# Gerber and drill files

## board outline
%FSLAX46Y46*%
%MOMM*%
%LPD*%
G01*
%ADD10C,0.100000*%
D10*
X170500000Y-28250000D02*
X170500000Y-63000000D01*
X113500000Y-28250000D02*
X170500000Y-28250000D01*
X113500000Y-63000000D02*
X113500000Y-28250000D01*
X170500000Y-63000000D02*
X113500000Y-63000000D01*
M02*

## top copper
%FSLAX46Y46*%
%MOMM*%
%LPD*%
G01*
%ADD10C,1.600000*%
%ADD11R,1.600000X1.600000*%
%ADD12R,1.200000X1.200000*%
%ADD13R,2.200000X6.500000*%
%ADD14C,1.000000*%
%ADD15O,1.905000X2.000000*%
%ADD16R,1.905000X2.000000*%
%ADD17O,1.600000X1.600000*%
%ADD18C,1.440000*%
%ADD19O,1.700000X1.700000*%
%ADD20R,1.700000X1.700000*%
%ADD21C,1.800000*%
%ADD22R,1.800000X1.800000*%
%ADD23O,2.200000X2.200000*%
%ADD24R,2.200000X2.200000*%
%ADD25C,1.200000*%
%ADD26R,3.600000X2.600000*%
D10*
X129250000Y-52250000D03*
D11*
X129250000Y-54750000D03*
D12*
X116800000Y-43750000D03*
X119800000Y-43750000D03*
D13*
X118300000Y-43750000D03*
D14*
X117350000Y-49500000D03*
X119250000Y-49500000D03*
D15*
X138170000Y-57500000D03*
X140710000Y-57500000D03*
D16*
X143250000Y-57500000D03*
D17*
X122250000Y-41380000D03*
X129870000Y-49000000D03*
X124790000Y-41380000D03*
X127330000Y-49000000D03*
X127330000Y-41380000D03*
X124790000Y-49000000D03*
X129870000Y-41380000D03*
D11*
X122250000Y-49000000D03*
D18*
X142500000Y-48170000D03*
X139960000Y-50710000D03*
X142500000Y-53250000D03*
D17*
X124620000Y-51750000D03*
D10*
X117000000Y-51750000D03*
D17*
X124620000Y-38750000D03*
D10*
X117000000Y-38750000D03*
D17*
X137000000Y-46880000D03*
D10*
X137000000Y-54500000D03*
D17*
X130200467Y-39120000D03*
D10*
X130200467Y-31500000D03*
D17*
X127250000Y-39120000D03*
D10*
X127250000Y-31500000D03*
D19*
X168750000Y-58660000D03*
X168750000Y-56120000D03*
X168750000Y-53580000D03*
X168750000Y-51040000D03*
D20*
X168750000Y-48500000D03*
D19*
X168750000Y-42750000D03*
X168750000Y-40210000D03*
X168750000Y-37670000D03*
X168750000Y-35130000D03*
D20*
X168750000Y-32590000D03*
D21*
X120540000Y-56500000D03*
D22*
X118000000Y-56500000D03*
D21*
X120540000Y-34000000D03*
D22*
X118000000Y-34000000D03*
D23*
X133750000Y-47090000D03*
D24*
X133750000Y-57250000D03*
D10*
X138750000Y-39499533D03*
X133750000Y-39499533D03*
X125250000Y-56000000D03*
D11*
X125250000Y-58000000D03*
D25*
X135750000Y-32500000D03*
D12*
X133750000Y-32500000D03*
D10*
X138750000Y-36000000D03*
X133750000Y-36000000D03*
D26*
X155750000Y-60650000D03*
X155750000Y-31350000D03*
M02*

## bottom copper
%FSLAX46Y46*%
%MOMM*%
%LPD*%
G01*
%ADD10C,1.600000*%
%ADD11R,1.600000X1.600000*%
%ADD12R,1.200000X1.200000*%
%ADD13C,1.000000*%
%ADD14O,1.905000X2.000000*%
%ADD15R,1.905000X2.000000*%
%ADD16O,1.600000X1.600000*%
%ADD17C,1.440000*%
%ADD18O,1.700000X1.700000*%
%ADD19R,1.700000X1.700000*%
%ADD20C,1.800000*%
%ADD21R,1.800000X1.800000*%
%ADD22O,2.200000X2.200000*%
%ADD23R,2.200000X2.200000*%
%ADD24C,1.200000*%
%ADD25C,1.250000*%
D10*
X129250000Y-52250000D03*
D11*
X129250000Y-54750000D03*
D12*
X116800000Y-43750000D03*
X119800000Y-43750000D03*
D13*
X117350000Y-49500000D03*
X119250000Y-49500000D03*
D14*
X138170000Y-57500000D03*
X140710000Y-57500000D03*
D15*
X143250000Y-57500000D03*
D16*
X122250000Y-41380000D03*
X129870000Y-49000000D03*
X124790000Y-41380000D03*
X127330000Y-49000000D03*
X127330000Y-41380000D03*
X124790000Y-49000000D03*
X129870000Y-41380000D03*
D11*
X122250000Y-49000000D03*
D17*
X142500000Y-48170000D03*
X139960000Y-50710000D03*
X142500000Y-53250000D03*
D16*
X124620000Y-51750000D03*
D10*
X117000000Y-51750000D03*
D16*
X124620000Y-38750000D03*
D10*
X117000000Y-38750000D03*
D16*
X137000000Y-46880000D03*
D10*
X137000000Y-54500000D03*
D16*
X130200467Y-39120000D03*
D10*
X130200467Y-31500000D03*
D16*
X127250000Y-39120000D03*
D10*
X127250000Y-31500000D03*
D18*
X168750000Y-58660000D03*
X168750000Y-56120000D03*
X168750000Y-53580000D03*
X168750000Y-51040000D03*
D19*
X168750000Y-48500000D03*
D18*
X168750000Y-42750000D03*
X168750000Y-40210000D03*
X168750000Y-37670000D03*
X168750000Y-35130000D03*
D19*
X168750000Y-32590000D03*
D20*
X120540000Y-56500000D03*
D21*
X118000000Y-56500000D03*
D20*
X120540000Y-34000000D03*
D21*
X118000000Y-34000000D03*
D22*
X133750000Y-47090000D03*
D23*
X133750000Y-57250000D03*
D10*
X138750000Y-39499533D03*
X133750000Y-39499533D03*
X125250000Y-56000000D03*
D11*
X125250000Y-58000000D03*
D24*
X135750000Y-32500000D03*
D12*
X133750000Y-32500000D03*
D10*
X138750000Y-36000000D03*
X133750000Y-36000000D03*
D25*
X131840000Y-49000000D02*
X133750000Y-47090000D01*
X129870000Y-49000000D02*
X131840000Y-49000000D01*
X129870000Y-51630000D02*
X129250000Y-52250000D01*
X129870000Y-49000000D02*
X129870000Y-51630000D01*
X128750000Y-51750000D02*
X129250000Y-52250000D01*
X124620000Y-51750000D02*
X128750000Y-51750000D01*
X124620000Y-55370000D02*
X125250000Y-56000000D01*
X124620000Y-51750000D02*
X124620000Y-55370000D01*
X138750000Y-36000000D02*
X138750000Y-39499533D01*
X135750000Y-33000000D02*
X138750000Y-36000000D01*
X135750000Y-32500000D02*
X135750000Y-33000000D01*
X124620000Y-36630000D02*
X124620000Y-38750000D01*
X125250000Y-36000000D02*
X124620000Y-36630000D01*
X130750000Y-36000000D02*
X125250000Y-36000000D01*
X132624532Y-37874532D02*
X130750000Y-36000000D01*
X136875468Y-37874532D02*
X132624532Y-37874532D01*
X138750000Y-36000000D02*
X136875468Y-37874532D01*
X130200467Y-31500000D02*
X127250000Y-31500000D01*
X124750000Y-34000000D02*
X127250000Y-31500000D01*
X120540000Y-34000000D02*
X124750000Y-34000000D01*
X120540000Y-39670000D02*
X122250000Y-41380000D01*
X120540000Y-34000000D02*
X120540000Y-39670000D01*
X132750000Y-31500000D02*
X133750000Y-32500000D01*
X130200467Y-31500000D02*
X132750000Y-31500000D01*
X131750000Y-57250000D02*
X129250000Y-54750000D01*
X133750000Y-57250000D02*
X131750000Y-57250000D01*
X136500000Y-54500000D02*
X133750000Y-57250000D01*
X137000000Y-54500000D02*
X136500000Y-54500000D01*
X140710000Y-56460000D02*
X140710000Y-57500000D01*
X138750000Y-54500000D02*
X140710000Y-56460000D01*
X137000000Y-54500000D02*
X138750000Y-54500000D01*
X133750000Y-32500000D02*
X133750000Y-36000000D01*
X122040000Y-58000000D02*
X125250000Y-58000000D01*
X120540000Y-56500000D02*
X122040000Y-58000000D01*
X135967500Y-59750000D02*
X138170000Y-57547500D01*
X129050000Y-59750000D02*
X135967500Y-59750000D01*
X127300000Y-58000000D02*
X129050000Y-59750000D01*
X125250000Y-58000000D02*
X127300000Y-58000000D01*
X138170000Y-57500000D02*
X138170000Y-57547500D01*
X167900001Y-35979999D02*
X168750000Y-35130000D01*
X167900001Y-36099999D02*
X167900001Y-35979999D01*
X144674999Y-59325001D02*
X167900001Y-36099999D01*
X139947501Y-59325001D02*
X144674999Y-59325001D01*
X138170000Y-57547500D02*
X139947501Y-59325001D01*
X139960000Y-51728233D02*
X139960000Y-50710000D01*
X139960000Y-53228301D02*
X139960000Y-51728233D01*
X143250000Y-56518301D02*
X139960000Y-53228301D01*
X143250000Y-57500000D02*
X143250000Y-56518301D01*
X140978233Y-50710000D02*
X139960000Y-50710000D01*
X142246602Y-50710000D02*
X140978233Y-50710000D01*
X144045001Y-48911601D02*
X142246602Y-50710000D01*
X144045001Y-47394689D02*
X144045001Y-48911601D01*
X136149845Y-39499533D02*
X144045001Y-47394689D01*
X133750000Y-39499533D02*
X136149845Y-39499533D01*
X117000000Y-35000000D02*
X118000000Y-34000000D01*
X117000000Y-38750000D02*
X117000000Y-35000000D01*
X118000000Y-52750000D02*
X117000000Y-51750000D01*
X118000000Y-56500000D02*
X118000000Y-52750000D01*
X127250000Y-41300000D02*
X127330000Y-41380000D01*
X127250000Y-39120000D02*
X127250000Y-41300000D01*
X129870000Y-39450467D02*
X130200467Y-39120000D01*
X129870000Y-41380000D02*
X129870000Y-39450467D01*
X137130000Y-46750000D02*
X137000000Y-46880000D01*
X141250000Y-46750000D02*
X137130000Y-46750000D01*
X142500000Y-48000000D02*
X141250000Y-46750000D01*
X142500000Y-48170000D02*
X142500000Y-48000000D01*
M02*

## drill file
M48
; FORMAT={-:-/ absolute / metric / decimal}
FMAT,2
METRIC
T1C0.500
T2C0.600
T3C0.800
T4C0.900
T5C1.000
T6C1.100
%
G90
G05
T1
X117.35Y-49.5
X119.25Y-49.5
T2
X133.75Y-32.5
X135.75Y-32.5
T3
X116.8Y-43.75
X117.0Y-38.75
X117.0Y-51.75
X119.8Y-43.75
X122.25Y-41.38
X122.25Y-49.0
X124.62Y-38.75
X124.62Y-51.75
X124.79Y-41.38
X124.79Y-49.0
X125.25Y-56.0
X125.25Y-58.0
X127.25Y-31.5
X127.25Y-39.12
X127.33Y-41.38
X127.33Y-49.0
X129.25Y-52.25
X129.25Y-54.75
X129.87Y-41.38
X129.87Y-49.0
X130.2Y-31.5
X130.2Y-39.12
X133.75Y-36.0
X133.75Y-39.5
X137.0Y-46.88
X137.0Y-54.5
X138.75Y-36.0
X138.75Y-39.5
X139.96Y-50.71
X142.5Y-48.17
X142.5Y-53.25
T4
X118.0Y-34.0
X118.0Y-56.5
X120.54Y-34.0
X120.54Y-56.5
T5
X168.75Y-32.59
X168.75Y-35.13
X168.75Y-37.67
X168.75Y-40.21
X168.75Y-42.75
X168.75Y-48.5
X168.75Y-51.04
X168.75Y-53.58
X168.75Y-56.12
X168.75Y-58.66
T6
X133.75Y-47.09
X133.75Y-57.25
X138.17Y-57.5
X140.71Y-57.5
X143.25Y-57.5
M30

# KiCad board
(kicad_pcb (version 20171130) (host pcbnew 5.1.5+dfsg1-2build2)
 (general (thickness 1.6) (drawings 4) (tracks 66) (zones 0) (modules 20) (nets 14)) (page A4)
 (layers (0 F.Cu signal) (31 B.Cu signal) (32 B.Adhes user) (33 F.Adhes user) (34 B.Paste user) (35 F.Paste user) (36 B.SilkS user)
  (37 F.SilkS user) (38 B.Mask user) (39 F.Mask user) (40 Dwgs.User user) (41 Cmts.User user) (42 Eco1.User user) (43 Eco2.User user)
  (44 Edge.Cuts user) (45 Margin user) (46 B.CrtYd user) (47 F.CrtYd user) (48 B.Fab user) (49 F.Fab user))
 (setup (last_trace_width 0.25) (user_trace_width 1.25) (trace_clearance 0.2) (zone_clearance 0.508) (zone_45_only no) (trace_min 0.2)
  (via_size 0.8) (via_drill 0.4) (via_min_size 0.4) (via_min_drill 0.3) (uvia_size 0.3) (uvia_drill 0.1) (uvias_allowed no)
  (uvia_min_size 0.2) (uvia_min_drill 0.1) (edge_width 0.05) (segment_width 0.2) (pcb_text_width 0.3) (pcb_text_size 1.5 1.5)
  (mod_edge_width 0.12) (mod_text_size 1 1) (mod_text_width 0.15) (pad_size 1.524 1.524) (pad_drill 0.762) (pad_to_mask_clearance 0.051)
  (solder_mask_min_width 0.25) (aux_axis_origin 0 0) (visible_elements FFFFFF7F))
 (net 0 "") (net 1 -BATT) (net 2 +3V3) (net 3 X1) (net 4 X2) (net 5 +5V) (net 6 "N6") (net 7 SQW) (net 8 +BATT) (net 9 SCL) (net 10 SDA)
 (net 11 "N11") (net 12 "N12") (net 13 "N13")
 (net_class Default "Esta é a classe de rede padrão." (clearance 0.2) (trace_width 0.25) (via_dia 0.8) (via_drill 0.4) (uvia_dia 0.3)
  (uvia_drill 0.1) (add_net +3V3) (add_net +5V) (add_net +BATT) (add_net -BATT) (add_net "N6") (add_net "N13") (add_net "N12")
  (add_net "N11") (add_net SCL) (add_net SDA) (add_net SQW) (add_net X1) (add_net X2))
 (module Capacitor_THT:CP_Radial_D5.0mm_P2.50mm (layer F.Cu) (at 129.25 54.75 90)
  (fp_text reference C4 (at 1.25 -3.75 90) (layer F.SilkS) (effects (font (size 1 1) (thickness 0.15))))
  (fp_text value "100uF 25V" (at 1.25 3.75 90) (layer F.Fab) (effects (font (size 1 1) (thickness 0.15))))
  (pad 2 thru_hole circle (at 2.5 0 90) (size 1.6 1.6) (drill 0.8) (layers *.Cu *.Mask) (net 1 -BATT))
  (pad 1 thru_hole rect (at 0 0 90) (size 1.6 1.6) (drill 0.8) (layers *.Cu *.Mask) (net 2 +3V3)))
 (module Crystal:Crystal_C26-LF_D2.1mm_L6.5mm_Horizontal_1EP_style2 (layer F.Cu) (at 119.25 49.5 180)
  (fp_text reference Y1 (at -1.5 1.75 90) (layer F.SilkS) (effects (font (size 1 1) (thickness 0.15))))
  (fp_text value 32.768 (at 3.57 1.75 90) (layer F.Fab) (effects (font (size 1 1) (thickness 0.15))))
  (pad 3 thru_hole rect (at 2.45 5.75 180) (size 1.2 1.2) (drill 0.8) (layers *.Cu *.Mask))
  (pad 3 thru_hole rect (at -0.55 5.75 180) (size 1.2 1.2) (drill 0.8) (layers *.Cu *.Mask))
  (pad 3 smd rect (at 0.95 5.75 180) (size 2.2 6.5) (layers F.Cu F.Paste F.Mask))
  (pad 2 thru_hole circle (at 1.9 0 180) (size 1 1) (drill 0.5) (layers *.Cu *.Mask) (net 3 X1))
  (pad 1 thru_hole circle (at 0 0 180) (size 1 1) (drill 0.5) (layers *.Cu *.Mask) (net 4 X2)))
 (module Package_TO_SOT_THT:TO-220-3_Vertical (layer F.Cu) (at 143.25 57.5 180)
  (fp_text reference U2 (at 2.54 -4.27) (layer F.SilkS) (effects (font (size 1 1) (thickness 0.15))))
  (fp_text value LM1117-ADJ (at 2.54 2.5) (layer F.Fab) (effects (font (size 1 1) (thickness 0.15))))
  (pad 3 thru_hole oval (at 5.08 0 180) (size 1.905 2) (drill 1.1) (layers *.Cu *.Mask) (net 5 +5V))
  (pad 2 thru_hole oval (at 2.54 0 180) (size 1.905 2) (drill 1.1) (layers *.Cu *.Mask) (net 2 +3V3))
  (pad 1 thru_hole rect (at 0 0 180) (size 1.905 2) (drill 1.1) (layers *.Cu *.Mask) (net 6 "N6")))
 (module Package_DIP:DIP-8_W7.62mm (layer F.Cu) (at 122.25 49 90)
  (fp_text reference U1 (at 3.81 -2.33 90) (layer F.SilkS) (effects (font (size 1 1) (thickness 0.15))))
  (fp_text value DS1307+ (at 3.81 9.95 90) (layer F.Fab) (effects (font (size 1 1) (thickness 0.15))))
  (pad 8 thru_hole oval (at 7.62 0 90) (size 1.6 1.6) (drill 0.8) (layers *.Cu *.Mask) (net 2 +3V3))
  (pad 4 thru_hole oval (at 0 7.62 90) (size 1.6 1.6) (drill 0.8) (layers *.Cu *.Mask) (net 1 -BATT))
  (pad 7 thru_hole oval (at 7.62 2.54 90) (size 1.6 1.6) (drill 0.8) (layers *.Cu *.Mask) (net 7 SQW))
  (pad 3 thru_hole oval (at 0 5.08 90) (size 1.6 1.6) (drill 0.8) (layers *.Cu *.Mask) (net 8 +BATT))
  (pad 6 thru_hole oval (at 7.62 5.08 90) (size 1.6 1.6) (drill 0.8) (layers *.Cu *.Mask) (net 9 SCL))
  (pad 2 thru_hole oval (at 0 2.54 90) (size 1.6 1.6) (drill 0.8) (layers *.Cu *.Mask) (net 4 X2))
  (pad 5 thru_hole oval (at 7.62 7.62 90) (size 1.6 1.6) (drill 0.8) (layers *.Cu *.Mask) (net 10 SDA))
  (pad 1 thru_hole rect (at 0 0 90) (size 1.6 1.6) (drill 0.8) (layers *.Cu *.Mask) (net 3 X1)))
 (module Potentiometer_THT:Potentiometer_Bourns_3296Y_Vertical (layer F.Cu) (at 142.5 53.25 270)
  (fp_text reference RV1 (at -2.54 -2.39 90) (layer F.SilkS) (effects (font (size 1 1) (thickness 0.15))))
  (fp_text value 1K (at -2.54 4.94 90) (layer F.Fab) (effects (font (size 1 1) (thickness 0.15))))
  (pad 3 thru_hole circle (at -5.08 0 270) (size 1.44 1.44) (drill 0.8) (layers *.Cu *.Mask) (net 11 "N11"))
  (pad 2 thru_hole circle (at -2.54 2.54 270) (size 1.44 1.44) (drill 0.8) (layers *.Cu *.Mask) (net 6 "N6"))
  (pad 1 thru_hole circle (at 0 0 270) (size 1.44 1.44) (drill 0.8) (layers *.Cu *.Mask) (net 1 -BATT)))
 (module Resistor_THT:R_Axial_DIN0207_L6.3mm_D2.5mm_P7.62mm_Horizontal (layer F.Cu) (at 117 51.75)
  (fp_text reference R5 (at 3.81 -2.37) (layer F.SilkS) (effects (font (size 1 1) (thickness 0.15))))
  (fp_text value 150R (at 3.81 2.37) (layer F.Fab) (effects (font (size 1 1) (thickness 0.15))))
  (pad 2 thru_hole oval (at 7.62 0) (size 1.6 1.6) (drill 0.8) (layers *.Cu *.Mask) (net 1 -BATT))
  (pad 1 thru_hole circle (at 0 0) (size 1.6 1.6) (drill 0.8) (layers *.Cu *.Mask) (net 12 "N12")))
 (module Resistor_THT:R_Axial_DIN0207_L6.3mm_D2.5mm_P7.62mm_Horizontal (layer F.Cu) (at 117 38.75)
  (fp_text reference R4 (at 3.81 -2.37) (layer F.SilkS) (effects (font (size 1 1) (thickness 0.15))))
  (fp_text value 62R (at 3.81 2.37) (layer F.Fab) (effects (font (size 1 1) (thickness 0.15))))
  (pad 2 thru_hole oval (at 7.62 0) (size 1.6 1.6) (drill 0.8) (layers *.Cu *.Mask) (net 1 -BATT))
  (pad 1 thru_hole circle (at 0 0) (size 1.6 1.6) (drill 0.8) (layers *.Cu *.Mask) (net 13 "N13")))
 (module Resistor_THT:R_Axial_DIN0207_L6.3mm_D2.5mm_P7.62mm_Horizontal (layer F.Cu) (at 137 54.5 90)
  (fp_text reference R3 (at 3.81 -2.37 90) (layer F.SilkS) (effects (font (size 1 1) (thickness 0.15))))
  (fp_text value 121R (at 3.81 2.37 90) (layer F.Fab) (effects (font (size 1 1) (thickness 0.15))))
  (pad 2 thru_hole oval (at 7.62 0 90) (size 1.6 1.6) (drill 0.8) (layers *.Cu *.Mask) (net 11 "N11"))
  (pad 1 thru_hole circle (at 0 0 90) (size 1.6 1.6) (drill 0.8) (layers *.Cu *.Mask) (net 2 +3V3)))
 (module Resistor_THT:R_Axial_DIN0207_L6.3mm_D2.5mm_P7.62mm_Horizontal (layer F.Cu) (at 130.200467 31.5 270)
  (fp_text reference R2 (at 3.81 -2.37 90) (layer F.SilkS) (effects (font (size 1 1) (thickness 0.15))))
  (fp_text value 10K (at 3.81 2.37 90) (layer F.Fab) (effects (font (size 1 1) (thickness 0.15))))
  (pad 2 thru_hole oval (at 7.62 0 270) (size 1.6 1.6) (drill 0.8) (layers *.Cu *.Mask) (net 10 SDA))
  (pad 1 thru_hole circle (at 0 0 270) (size 1.6 1.6) (drill 0.8) (layers *.Cu *.Mask) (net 2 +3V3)))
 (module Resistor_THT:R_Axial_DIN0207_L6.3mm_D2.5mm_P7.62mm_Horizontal (layer F.Cu) (at 127.25 31.5 270)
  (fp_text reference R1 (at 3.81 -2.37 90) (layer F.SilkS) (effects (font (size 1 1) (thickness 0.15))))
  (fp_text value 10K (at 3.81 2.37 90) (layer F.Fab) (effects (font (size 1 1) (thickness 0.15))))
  (pad 2 thru_hole oval (at 7.62 0 270) (size 1.6 1.6) (drill 0.8) (layers *.Cu *.Mask) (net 9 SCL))
  (pad 1 thru_hole circle (at 0 0 270) (size 1.6 1.6) (drill 0.8) (layers *.Cu *.Mask) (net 2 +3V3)))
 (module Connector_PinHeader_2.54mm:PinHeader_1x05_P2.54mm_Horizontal (layer F.Cu) (at 168.75 48.5)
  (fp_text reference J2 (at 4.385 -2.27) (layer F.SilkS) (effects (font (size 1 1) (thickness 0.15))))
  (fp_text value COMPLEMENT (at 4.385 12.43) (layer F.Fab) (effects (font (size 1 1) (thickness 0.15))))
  (pad 5 thru_hole oval (at 0 10.16) (size 1.7 1.7) (drill 1) (layers *.Cu *.Mask) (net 4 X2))
  (pad 4 thru_hole oval (at 0 7.62) (size 1.7 1.7) (drill 1) (layers *.Cu *.Mask) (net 3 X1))
  (pad 3 thru_hole oval (at 0 5.08) (size 1.7 1.7) (drill 1) (layers *.Cu *.Mask) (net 8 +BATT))
  (pad 2 thru_hole oval (at 0 2.54) (size 1.7 1.7) (drill 1) (layers *.Cu *.Mask) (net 2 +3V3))
  (pad 1 thru_hole rect (at 0 0) (size 1.7 1.7) (drill 1) (layers *.Cu *.Mask) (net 1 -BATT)))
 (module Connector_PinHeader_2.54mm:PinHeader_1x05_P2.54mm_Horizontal (layer F.Cu) (at 168.75 32.59)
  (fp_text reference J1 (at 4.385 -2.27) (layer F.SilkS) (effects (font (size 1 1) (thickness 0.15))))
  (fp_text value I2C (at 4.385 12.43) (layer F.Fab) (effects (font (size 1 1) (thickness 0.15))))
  (pad 5 thru_hole oval (at 0 10.16) (size 1.7 1.7) (drill 1) (layers *.Cu *.Mask) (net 7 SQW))
  (pad 4 thru_hole oval (at 0 7.62) (size 1.7 1.7) (drill 1) (layers *.Cu *.Mask) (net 9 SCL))
  (pad 3 thru_hole oval (at 0 5.08) (size 1.7 1.7) (drill 1) (layers *.Cu *.Mask) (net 10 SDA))
  (pad 2 thru_hole oval (at 0 2.54) (size 1.7 1.7) (drill 1) (layers *.Cu *.Mask) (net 5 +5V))
  (pad 1 thru_hole rect (at 0 0) (size 1.7 1.7) (drill 1) (layers *.Cu *.Mask) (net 1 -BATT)))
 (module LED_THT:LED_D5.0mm (layer F.Cu) (at 118 56.5)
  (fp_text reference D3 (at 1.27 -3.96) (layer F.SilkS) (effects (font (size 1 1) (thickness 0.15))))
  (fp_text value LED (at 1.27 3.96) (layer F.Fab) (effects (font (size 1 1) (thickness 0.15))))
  (pad 2 thru_hole circle (at 2.54 0) (size 1.8 1.8) (drill 0.9) (layers *.Cu *.Mask) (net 5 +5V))
  (pad 1 thru_hole rect (at 0 0) (size 1.8 1.8) (drill 0.9) (layers *.Cu *.Mask) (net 12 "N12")))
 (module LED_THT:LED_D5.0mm (layer F.Cu) (at 118 34)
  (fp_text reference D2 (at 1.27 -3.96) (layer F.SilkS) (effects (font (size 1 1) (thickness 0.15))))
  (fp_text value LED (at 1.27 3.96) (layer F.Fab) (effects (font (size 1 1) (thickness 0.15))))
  (pad 2 thru_hole circle (at 2.54 0) (size 1.8 1.8) (drill 0.9) (layers *.Cu *.Mask) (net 2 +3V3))
  (pad 1 thru_hole rect (at 0 0) (size 1.8 1.8) (drill 0.9) (layers *.Cu *.Mask) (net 13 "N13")))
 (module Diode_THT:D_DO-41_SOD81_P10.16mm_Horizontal (layer F.Cu) (at 133.75 57.25 90)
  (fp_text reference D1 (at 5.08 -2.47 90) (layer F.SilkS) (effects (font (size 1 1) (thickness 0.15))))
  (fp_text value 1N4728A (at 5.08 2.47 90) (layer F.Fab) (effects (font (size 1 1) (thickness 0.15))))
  (pad 2 thru_hole oval (at 10.16 0 90) (size 2.2 2.2) (drill 1.1) (layers *.Cu *.Mask) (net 1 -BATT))
  (pad 1 thru_hole rect (at 0 0 90) (size 2.2 2.2) (drill 1.1) (layers *.Cu *.Mask) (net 2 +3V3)))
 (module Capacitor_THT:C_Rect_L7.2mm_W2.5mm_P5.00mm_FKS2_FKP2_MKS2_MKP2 (layer F.Cu) (at 133.75 39.499533)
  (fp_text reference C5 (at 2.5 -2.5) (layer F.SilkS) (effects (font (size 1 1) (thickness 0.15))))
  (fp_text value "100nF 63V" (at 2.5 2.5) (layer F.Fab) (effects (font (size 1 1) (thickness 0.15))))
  (pad 2 thru_hole circle (at 5 0) (size 1.6 1.6) (drill 0.8) (layers *.Cu *.Mask) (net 1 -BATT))
  (pad 1 thru_hole circle (at 0 0) (size 1.6 1.6) (drill 0.8) (layers *.Cu *.Mask) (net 6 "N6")))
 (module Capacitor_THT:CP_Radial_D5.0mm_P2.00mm (layer F.Cu) (at 125.25 58 90)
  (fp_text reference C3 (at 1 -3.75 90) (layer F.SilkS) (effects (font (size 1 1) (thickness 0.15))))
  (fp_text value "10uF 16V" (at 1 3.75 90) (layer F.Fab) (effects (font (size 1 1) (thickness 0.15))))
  (pad 2 thru_hole circle (at 2 0 90) (size 1.6 1.6) (drill 0.8) (layers *.Cu *.Mask) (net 1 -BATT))
  (pad 1 thru_hole rect (at 0 0 90) (size 1.6 1.6) (drill 0.8) (layers *.Cu *.Mask) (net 5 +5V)))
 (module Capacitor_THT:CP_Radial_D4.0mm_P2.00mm (layer F.Cu) (at 133.75 32.5)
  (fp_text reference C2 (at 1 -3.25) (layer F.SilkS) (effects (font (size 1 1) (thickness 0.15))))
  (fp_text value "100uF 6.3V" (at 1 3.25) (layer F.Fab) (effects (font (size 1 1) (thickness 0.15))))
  (pad 2 thru_hole circle (at 2 0) (size 1.2 1.2) (drill 0.6) (layers *.Cu *.Mask) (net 1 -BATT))
  (pad 1 thru_hole rect (at 0 0) (size 1.2 1.2) (drill 0.6) (layers *.Cu *.Mask) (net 2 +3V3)))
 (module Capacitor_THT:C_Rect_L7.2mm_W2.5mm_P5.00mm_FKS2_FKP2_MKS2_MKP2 (layer F.Cu) (at 133.75 36)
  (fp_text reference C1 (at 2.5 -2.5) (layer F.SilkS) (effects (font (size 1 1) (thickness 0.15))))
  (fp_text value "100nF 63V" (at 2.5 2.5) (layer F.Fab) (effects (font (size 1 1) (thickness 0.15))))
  (pad 2 thru_hole circle (at 5 0) (size 1.6 1.6) (drill 0.8) (layers *.Cu *.Mask) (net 1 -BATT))
  (pad 1 thru_hole circle (at 0 0) (size 1.6 1.6) (drill 0.8) (layers *.Cu *.Mask) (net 2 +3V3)))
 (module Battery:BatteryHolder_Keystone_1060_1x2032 (layer F.Cu) (at 155.75 46 90)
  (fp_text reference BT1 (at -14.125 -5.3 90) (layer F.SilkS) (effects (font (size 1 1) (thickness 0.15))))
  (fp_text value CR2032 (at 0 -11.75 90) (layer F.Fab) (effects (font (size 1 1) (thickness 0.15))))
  (pad 1 smd rect (at -14.65 0 270) (size 2.6 3.6) (layers F.Cu F.Paste F.Mask) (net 8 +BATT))
  (pad 2 smd rect (at 14.65 0 270) (size 2.6 3.6) (layers F.Cu F.Paste F.Mask) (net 1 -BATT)))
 (gr_line (start 170.5 28.25) (end 170.5 63) (layer Edge.Cuts) (width 0.1))
 (gr_line (start 113.5 28.25) (end 170.5 28.25) (layer Edge.Cuts) (width 0.1))
 (gr_line (start 113.5 63) (end 113.5 28.25) (layer Edge.Cuts) (width 0.1))
 (gr_line (start 170.5 63) (end 113.5 63) (layer Edge.Cuts) (width 0.1))
 (segment (start 131.84 49) (end 133.75 47.09) (width 1.25) (layer B.Cu) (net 1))
 (segment (start 129.87 49) (end 131.84 49) (width 1.25) (layer B.Cu) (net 1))
 (segment (start 129.87 51.63) (end 129.25 52.25) (width 1.25) (layer B.Cu) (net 1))
 (segment (start 129.87 49) (end 129.87 51.63) (width 1.25) (layer B.Cu) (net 1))
 (segment (start 128.75 51.75) (end 129.25 52.25) (width 1.25) (layer B.Cu) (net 1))
 (segment (start 124.62 51.75) (end 128.75 51.75) (width 1.25) (layer B.Cu) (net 1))
 (segment (start 124.62 55.37) (end 125.25 56) (width 1.25) (layer B.Cu) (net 1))
 (segment (start 124.62 51.75) (end 124.62 55.37) (width 1.25) (layer B.Cu) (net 1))
 (segment (start 138.75 36) (end 138.75 39.499533) (width 1.25) (layer B.Cu) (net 1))
 (segment (start 135.75 33) (end 138.75 36) (width 1.25) (layer B.Cu) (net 1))
 (segment (start 135.75 32.5) (end 135.75 33) (width 1.25) (layer B.Cu) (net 1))
 (segment (start 124.62 36.63) (end 124.62 38.75) (width 1.25) (layer B.Cu) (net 1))
 (segment (start 125.25 36) (end 124.62 36.63) (width 1.25) (layer B.Cu) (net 1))
 (segment (start 130.75 36) (end 125.25 36) (width 1.25) (layer B.Cu) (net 1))
 (segment (start 132.624532 37.874532) (end 130.75 36) (width 1.25) (layer B.Cu) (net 1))
 (segment (start 136.875468 37.874532) (end 132.624532 37.874532) (width 1.25) (layer B.Cu) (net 1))
 (segment (start 138.75 36) (end 136.875468 37.874532) (width 1.25) (layer B.Cu) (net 1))
 (segment (start 130.200467 31.5) (end 127.25 31.5) (width 1.25) (layer B.Cu) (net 2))
 (segment (start 124.75 34) (end 127.25 31.5) (width 1.25) (layer B.Cu) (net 2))
 (segment (start 120.54 34) (end 124.75 34) (width 1.25) (layer B.Cu) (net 2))
 (segment (start 120.54 39.67) (end 122.25 41.38) (width 1.25) (layer B.Cu) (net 2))
 (segment (start 120.54 34) (end 120.54 39.67) (width 1.25) (layer B.Cu) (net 2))
 (segment (start 132.75 31.5) (end 133.75 32.5) (width 1.25) (layer B.Cu) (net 2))
 (segment (start 130.200467 31.5) (end 132.75 31.5) (width 1.25) (layer B.Cu) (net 2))
 (segment (start 131.75 57.25) (end 129.25 54.75) (width 1.25) (layer B.Cu) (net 2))
 (segment (start 133.75 57.25) (end 131.75 57.25) (width 1.25) (layer B.Cu) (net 2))
 (segment (start 136.5 54.5) (end 133.75 57.25) (width 1.25) (layer B.Cu) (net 2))
 (segment (start 137 54.5) (end 136.5 54.5) (width 1.25) (layer B.Cu) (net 2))
 (segment (start 140.71 56.46) (end 140.71 57.5) (width 1.25) (layer B.Cu) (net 2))
 (segment (start 138.75 54.5) (end 140.71 56.46) (width 1.25) (layer B.Cu) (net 2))
 (segment (start 137 54.5) (end 138.75 54.5) (width 1.25) (layer B.Cu) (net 2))
 (segment (start 133.75 32.5) (end 133.75 36) (width 1.25) (layer B.Cu) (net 2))
 (segment (start 122.04 58) (end 125.25 58) (width 1.25) (layer B.Cu) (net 5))
 (segment (start 120.54 56.5) (end 122.04 58) (width 1.25) (layer B.Cu) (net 5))
 (segment (start 135.9675 59.75) (end 138.17 57.5475) (width 1.25) (layer B.Cu) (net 5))
 (segment (start 129.05 59.75) (end 135.9675 59.75) (width 1.25) (layer B.Cu) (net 5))
 (segment (start 127.3 58) (end 129.05 59.75) (width 1.25) (layer B.Cu) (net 5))
 (segment (start 125.25 58) (end 127.3 58) (width 1.25) (layer B.Cu) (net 5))
 (segment (start 138.17 57.5) (end 138.17 57.5475) (width 1.25) (layer B.Cu) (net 5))
 (segment (start 167.900001 35.979999) (end 168.75 35.13) (width 1.25) (layer B.Cu) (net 5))
 (segment (start 167.900001 36.099999) (end 167.900001 35.979999) (width 1.25) (layer B.Cu) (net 5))
 (segment (start 144.674999 59.325001) (end 167.900001 36.099999) (width 1.25) (layer B.Cu) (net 5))
 (segment (start 139.947501 59.325001) (end 144.674999 59.325001) (width 1.25) (layer B.Cu) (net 5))
 (segment (start 138.17 57.5475) (end 139.947501 59.325001) (width 1.25) (layer B.Cu) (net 5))
 (segment (start 139.96 51.728233) (end 139.96 50.71) (width 1.25) (layer B.Cu) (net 6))
 (segment (start 139.96 53.228301) (end 139.96 51.728233) (width 1.25) (layer B.Cu) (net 6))
 (segment (start 143.25 56.518301) (end 139.96 53.228301) (width 1.25) (layer B.Cu) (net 6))
 (segment (start 143.25 57.5) (end 143.25 56.518301) (width 1.25) (layer B.Cu) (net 6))
 (segment (start 140.978233 50.71) (end 139.96 50.71) (width 1.25) (layer B.Cu) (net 6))
 (segment (start 142.246602 50.71) (end 140.978233 50.71) (width 1.25) (layer B.Cu) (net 6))
 (segment (start 144.045001 48.911601) (end 142.246602 50.71) (width 1.25) (layer B.Cu) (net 6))
 (segment (start 144.045001 47.394689) (end 144.045001 48.911601) (width 1.25) (layer B.Cu) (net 6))
 (segment (start 136.149845 39.499533) (end 144.045001 47.394689) (width 1.25) (layer B.Cu) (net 6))
 (segment (start 133.75 39.499533) (end 136.149845 39.499533) (width 1.25) (layer B.Cu) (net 6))
 (segment (start 117 35) (end 118 34) (width 1.25) (layer B.Cu) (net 13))
 (segment (start 117 38.75) (end 117 35) (width 1.25) (layer B.Cu) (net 13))
 (segment (start 118 52.75) (end 117 51.75) (width 1.25) (layer B.Cu) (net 12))
 (segment (start 118 56.5) (end 118 52.75) (width 1.25) (layer B.Cu) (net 12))
 (segment (start 127.25 41.3) (end 127.33 41.38) (width 1.25) (layer B.Cu) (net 9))
 (segment (start 127.25 39.12) (end 127.25 41.3) (width 1.25) (layer B.Cu) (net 9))
 (segment (start 129.87 39.450467) (end 130.200467 39.12) (width 1.25) (layer B.Cu) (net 10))
 (segment (start 129.87 41.38) (end 129.87 39.450467) (width 1.25) (layer B.Cu) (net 10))
 (segment (start 137.13 46.75) (end 137 46.88) (width 1.25) (layer B.Cu) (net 11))
 (segment (start 141.25 46.75) (end 137.13 46.75) (width 1.25) (layer B.Cu) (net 11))
 (segment (start 142.5 48) (end 141.25 46.75) (width 1.25) (layer B.Cu) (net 11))
 (segment (start 142.5 48.17) (end 142.5 48) (width 1.25) (layer B.Cu) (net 11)))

